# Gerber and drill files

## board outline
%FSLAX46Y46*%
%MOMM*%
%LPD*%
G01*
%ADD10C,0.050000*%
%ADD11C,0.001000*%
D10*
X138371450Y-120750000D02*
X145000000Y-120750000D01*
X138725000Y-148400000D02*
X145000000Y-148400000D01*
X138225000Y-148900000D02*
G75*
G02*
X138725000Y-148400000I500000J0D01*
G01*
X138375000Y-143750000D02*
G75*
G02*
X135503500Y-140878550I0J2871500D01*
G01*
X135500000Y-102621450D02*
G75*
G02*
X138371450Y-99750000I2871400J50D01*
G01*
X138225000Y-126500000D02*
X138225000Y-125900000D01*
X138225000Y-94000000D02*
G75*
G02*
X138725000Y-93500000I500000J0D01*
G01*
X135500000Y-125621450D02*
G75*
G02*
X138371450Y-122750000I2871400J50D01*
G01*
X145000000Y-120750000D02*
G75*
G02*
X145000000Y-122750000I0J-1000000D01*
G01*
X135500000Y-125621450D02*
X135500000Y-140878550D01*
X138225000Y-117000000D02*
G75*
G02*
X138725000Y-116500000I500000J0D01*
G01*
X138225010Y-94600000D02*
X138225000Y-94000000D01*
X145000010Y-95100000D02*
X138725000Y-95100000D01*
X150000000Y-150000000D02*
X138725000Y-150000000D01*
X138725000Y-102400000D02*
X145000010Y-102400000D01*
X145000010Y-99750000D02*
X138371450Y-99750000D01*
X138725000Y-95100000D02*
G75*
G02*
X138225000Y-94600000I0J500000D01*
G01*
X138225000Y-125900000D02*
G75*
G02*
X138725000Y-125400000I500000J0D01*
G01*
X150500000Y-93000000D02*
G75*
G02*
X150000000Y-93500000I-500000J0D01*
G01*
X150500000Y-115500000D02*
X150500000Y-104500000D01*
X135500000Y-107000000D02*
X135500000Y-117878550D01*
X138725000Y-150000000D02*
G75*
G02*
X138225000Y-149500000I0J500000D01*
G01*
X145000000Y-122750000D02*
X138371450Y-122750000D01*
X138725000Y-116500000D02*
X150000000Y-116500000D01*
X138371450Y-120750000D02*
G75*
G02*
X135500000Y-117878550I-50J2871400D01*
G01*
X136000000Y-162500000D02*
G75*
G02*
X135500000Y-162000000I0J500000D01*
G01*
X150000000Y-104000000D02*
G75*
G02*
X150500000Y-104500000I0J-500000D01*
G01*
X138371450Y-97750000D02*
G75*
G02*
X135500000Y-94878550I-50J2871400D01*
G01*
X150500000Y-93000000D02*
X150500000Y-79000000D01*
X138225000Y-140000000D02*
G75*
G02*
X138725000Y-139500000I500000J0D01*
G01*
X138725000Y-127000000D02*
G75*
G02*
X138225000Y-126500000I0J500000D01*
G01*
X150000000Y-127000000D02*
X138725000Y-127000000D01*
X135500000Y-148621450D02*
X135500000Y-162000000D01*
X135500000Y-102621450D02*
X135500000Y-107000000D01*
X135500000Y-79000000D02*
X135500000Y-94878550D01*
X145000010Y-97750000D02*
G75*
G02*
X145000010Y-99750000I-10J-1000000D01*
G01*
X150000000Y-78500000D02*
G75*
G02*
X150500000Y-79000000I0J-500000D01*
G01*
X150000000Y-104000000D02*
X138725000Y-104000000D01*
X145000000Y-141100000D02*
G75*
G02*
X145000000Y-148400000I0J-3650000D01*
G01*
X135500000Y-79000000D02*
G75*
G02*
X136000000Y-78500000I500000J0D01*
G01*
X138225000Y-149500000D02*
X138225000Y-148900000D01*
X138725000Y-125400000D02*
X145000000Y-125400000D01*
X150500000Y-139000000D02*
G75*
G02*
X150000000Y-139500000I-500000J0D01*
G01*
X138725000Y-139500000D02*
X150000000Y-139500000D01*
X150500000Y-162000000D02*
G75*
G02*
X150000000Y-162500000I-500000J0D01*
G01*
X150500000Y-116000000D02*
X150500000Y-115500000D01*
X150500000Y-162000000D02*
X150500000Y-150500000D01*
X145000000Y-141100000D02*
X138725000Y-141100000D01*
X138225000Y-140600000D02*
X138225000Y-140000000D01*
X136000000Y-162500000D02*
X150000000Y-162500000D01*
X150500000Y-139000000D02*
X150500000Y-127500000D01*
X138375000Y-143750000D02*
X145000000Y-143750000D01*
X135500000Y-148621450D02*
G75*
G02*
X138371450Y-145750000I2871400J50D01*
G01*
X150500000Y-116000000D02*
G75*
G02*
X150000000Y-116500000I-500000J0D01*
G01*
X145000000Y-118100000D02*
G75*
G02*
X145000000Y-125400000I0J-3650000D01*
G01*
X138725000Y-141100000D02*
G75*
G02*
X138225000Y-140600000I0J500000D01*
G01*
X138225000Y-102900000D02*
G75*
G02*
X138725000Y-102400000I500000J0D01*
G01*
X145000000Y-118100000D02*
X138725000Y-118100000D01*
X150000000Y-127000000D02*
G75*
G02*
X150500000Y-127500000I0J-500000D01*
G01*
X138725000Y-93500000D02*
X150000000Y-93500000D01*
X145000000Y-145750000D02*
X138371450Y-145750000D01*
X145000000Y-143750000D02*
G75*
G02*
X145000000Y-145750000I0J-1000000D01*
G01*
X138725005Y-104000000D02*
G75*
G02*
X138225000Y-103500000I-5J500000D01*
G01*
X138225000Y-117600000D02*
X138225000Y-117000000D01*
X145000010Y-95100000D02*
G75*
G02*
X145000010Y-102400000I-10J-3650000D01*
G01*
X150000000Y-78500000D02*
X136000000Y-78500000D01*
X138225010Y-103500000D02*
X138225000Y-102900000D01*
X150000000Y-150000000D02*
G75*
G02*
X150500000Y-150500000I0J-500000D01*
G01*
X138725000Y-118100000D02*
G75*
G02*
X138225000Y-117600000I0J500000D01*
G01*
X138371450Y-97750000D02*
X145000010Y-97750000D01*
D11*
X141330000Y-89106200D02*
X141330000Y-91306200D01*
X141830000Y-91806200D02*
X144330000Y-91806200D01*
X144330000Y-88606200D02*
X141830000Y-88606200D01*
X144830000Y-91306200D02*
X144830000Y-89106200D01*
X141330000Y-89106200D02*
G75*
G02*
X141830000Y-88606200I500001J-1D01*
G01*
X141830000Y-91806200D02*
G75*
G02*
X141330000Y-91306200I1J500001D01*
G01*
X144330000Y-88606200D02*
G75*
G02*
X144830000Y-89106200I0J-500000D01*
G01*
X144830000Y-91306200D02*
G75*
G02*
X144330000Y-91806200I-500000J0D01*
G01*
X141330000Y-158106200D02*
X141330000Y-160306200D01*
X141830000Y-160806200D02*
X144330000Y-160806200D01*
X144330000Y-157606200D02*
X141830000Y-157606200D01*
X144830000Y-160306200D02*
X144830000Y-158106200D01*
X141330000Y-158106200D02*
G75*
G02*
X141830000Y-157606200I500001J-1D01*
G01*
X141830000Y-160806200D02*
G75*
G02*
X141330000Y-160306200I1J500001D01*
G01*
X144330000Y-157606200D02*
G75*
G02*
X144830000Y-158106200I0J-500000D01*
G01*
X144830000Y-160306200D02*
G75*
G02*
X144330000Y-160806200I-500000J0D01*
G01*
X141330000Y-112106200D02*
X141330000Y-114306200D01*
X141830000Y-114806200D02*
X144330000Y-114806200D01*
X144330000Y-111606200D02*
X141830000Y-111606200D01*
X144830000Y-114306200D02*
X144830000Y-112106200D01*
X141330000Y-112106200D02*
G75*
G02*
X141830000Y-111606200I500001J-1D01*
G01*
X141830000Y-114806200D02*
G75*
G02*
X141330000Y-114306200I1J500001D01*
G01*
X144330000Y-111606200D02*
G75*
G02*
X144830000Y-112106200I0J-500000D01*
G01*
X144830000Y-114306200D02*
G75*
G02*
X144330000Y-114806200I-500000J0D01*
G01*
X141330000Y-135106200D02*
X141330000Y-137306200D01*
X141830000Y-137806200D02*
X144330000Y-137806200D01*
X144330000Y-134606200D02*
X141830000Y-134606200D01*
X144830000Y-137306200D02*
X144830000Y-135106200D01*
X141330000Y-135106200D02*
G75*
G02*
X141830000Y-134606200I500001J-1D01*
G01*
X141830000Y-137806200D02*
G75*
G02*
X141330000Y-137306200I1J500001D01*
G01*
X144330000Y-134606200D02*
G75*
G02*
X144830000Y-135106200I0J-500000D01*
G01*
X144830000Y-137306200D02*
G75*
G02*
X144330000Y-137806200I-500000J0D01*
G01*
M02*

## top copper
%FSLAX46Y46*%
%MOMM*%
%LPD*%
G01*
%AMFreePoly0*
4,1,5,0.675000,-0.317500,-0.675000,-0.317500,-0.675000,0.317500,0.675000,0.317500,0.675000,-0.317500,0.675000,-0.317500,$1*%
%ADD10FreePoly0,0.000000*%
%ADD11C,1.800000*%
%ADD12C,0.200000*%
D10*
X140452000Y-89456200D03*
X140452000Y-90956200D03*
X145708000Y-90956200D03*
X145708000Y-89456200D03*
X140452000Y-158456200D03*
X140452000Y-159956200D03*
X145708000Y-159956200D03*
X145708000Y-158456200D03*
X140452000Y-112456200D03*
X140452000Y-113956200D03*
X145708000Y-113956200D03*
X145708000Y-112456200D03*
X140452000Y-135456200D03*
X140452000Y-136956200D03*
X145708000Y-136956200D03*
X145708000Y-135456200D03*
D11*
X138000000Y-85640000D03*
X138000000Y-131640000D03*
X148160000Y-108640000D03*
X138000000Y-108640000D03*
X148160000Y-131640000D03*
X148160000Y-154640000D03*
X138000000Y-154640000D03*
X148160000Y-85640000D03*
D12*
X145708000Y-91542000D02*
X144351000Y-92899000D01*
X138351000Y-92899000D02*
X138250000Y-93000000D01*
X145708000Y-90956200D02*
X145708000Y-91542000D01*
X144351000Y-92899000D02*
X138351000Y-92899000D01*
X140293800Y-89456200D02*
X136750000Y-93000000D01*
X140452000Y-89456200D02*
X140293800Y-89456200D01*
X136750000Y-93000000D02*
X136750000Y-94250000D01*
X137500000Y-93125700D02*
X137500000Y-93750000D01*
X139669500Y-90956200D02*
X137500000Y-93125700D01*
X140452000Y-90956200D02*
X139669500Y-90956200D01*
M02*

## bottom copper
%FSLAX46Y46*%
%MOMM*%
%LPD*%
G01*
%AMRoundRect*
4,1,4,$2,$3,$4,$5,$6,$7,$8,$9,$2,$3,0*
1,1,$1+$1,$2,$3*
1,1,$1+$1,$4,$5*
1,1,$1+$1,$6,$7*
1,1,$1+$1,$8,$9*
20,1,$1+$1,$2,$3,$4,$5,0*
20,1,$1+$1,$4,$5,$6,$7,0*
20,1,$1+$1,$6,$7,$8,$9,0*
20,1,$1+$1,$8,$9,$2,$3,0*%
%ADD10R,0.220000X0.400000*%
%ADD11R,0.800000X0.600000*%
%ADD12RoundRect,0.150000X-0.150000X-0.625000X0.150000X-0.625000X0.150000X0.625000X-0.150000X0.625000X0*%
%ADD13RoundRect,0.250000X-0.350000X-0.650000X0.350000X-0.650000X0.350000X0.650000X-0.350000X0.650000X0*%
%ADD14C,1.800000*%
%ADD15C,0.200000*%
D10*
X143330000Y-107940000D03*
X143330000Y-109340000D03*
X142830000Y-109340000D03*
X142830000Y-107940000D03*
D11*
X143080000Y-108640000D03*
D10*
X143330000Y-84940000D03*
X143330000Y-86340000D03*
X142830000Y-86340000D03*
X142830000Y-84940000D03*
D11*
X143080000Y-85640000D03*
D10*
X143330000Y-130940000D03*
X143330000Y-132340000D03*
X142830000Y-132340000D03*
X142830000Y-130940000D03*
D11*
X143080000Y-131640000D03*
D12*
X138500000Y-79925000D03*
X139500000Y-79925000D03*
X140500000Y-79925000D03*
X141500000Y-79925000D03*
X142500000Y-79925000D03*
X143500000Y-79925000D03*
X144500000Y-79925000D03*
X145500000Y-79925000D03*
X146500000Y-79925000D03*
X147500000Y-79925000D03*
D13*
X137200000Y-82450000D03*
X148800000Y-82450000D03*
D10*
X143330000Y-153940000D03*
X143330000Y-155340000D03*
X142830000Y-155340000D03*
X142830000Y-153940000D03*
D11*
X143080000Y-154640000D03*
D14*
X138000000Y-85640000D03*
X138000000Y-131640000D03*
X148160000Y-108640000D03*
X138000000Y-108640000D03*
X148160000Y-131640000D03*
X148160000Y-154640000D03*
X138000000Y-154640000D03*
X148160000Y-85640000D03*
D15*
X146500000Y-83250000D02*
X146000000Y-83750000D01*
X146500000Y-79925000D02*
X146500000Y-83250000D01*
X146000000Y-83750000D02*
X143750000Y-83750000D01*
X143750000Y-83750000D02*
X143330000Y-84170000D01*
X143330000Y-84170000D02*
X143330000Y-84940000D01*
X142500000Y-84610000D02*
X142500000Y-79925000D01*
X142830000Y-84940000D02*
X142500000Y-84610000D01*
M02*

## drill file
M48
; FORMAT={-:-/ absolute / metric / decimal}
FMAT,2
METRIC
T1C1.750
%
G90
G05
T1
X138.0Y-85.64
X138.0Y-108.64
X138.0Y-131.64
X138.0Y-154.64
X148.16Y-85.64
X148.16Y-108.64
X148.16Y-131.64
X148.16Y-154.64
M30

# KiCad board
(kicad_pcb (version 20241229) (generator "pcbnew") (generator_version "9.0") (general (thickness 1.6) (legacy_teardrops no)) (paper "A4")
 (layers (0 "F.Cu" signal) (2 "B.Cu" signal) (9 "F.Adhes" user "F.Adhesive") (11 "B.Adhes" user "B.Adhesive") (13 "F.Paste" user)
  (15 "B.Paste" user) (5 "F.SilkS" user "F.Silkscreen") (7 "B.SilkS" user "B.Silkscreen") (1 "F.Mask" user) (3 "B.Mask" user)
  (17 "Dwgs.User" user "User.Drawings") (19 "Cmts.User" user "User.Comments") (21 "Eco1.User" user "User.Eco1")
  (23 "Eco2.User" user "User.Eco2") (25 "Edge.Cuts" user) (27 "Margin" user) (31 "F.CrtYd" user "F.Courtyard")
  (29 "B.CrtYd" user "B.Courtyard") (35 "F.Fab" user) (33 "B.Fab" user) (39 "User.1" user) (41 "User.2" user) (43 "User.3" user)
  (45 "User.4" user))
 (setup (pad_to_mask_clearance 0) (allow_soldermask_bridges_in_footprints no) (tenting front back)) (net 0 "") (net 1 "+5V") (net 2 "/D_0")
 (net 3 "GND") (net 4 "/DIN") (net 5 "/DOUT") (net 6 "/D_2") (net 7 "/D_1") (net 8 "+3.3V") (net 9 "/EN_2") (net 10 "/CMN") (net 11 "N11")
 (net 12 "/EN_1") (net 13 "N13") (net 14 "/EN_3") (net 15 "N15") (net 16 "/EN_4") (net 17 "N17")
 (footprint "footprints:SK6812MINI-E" (layer "F.Cu") (at 143.08 90.2062)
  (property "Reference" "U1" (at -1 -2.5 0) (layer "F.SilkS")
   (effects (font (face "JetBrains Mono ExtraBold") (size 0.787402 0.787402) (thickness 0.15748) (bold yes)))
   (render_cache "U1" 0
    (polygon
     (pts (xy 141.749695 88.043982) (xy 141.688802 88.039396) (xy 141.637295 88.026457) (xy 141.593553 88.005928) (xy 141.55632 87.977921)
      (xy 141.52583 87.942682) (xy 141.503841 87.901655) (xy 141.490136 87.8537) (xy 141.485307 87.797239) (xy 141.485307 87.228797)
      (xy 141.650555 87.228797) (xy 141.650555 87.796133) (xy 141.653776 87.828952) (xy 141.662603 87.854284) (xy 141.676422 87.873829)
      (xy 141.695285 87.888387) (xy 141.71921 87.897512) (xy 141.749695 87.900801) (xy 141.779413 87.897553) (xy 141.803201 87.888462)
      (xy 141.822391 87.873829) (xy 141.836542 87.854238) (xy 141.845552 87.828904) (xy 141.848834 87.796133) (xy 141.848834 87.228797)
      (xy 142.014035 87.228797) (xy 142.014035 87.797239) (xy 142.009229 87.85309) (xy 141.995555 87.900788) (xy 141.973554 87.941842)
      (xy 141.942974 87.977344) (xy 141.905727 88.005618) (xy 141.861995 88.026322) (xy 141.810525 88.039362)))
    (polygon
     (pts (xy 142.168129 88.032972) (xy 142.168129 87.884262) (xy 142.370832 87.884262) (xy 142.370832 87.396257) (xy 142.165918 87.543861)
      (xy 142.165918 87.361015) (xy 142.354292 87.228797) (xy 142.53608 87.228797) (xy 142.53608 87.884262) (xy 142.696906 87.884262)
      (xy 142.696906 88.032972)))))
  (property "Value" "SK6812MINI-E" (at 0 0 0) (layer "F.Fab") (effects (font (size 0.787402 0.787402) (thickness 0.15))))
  (fp_line (start -1.75 -1.1) (end -1.75 1.1) (stroke (width 0.001) (type solid)) (layer "Edge.Cuts"))
  (fp_line (start -1.25 1.6) (end 1.25 1.6) (stroke (width 0.001) (type solid)) (layer "Edge.Cuts"))
  (fp_line (start 1.25 -1.6) (end -1.25 -1.6) (stroke (width 0.001) (type solid)) (layer "Edge.Cuts"))
  (fp_line (start 1.75 1.1) (end 1.75 -1.1) (stroke (width 0.001) (type solid)) (layer "Edge.Cuts"))
  (fp_arc (start -1.75 -1.1) (mid -1.603553 -1.453553) (end -1.25 -1.6) (stroke (width 0.001) (type default)) (layer "Edge.Cuts"))
  (fp_arc (start -1.25 1.6) (mid -1.603553 1.453553) (end -1.75 1.1) (stroke (width 0.001) (type default)) (layer "Edge.Cuts"))
  (fp_arc (start 1.25 -1.6) (mid 1.603553 -1.453553) (end 1.75 -1.1) (stroke (width 0.001) (type default)) (layer "Edge.Cuts"))
  (fp_arc (start 1.75 1.1) (mid 1.603553 1.453553) (end 1.25 1.6) (stroke (width 0.001) (type default)) (layer "Edge.Cuts"))
  (pad "P$1" smd custom (at -2.628 -0.75) (size 1.35 0.635) (layers "F.Cu" "F.Mask" "F.Paste") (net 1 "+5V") (solder_mask_margin 0.102)
   (options (clearance outline) (anchor rect)) (primitives))
  (pad "P$2" smd custom (at -2.628 0.75) (size 1.35 0.635) (layers "F.Cu" "F.Mask" "F.Paste") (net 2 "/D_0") (solder_mask_margin 0.102)
   (options (clearance outline) (anchor rect)) (primitives))
  (pad "P$3" smd custom (at 2.628 0.75) (size 1.35 0.635) (layers "F.Cu" "F.Mask" "F.Paste") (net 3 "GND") (solder_mask_margin 0.102)
   (options (clearance outline) (anchor rect)) (primitives))
  (pad "P$4" smd custom (at 2.628 -0.75) (size 1.35 0.635) (layers "F.Cu" "F.Mask" "F.Paste") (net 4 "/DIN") (solder_mask_margin 0.102)
   (options (clearance outline) (anchor rect)) (primitives)))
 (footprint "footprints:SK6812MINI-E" (layer "F.Cu") (at 143.08 159.2062)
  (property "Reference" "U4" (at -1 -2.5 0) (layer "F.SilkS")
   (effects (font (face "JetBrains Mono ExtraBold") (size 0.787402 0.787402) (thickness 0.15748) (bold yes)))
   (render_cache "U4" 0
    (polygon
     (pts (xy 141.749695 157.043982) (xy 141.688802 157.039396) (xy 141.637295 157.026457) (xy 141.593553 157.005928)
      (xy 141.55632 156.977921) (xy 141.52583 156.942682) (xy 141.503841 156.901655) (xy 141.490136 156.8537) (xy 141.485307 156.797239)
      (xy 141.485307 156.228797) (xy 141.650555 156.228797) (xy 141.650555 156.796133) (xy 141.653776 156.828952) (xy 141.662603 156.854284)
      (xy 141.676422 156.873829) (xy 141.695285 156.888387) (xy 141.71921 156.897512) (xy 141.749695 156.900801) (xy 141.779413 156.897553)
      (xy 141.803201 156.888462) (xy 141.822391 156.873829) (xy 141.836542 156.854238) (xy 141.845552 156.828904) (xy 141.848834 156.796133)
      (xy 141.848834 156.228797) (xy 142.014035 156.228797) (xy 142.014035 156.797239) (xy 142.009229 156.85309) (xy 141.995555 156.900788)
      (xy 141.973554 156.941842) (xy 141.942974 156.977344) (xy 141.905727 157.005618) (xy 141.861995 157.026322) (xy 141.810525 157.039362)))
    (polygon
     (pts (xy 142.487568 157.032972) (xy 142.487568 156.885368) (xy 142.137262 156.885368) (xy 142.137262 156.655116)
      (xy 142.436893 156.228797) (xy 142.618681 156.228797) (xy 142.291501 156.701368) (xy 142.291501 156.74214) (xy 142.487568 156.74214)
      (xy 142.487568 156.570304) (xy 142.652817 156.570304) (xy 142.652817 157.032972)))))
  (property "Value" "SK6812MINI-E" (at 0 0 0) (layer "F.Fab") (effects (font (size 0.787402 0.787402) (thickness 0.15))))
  (fp_line (start -1.75 -1.1) (end -1.75 1.1) (stroke (width 0.001) (type solid)) (layer "Edge.Cuts"))
  (fp_line (start -1.25 1.6) (end 1.25 1.6) (stroke (width 0.001) (type solid)) (layer "Edge.Cuts"))
  (fp_line (start 1.25 -1.6) (end -1.25 -1.6) (stroke (width 0.001) (type solid)) (layer "Edge.Cuts"))
  (fp_line (start 1.75 1.1) (end 1.75 -1.1) (stroke (width 0.001) (type solid)) (layer "Edge.Cuts"))
  (fp_arc (start -1.75 -1.1) (mid -1.603553 -1.453553) (end -1.25 -1.6) (stroke (width 0.001) (type default)) (layer "Edge.Cuts"))
  (fp_arc (start -1.25 1.6) (mid -1.603553 1.453553) (end -1.75 1.1) (stroke (width 0.001) (type default)) (layer "Edge.Cuts"))
  (fp_arc (start 1.25 -1.6) (mid 1.603553 -1.453553) (end 1.75 -1.1) (stroke (width 0.001) (type default)) (layer "Edge.Cuts"))
  (fp_arc (start 1.75 1.1) (mid 1.603553 1.453553) (end 1.25 1.6) (stroke (width 0.001) (type default)) (layer "Edge.Cuts"))
  (pad "P$1" smd custom (at -2.628 -0.75) (size 1.35 0.635) (layers "F.Cu" "F.Mask" "F.Paste") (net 1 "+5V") (solder_mask_margin 0.102)
   (options (clearance outline) (anchor rect)) (primitives))
  (pad "P$2" smd custom (at -2.628 0.75) (size 1.35 0.635) (layers "F.Cu" "F.Mask" "F.Paste") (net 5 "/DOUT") (solder_mask_margin 0.102)
   (options (clearance outline) (anchor rect)) (primitives))
  (pad "P$3" smd custom (at 2.628 0.75) (size 1.35 0.635) (layers "F.Cu" "F.Mask" "F.Paste") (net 3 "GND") (solder_mask_margin 0.102)
   (options (clearance outline) (anchor rect)) (primitives))
  (pad "P$4" smd custom (at 2.628 -0.75) (size 1.35 0.635) (layers "F.Cu" "F.Mask" "F.Paste") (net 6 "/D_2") (solder_mask_margin 0.102)
   (options (clearance outline) (anchor rect)) (primitives)))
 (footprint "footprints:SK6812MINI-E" (layer "F.Cu") (at 143.08 113.2062)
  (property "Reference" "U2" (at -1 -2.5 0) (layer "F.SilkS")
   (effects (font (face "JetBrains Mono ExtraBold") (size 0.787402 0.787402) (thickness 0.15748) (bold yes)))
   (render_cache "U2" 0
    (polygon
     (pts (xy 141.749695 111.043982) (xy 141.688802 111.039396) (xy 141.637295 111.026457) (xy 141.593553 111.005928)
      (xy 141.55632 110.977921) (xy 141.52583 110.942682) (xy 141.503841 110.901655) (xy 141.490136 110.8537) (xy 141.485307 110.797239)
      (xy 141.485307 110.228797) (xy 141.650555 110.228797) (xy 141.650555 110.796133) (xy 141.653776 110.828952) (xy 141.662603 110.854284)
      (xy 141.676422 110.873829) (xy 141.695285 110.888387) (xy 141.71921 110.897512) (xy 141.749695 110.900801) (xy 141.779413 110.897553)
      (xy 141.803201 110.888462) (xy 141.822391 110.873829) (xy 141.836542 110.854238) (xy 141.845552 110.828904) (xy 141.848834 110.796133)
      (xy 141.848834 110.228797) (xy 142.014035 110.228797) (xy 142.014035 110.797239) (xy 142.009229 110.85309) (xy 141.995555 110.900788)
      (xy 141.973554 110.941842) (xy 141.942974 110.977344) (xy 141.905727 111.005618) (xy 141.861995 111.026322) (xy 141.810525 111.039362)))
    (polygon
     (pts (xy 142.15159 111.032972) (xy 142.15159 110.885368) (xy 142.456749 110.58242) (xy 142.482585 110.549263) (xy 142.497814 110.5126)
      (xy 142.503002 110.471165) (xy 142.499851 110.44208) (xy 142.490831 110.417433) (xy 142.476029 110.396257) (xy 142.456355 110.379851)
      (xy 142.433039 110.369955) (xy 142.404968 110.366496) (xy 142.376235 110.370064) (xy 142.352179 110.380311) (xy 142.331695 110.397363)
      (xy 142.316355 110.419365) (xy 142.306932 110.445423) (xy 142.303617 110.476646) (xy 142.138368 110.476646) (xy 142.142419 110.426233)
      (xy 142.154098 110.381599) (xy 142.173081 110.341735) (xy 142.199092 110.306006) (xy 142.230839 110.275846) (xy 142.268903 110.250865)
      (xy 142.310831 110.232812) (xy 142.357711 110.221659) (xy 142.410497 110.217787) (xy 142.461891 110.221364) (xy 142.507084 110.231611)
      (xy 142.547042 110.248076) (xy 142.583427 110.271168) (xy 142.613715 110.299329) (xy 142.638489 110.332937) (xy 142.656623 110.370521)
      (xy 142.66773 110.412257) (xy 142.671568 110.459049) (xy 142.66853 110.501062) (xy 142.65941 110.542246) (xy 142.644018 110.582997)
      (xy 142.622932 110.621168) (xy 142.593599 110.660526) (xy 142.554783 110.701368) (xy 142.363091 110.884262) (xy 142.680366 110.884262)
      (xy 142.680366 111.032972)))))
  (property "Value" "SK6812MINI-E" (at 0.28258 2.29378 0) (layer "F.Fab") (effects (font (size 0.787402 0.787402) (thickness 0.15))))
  (fp_line (start -1.75 -1.1) (end -1.75 1.1) (stroke (width 0.001) (type solid)) (layer "Edge.Cuts"))
  (fp_line (start -1.25 1.6) (end 1.25 1.6) (stroke (width 0.001) (type solid)) (layer "Edge.Cuts"))
  (fp_line (start 1.25 -1.6) (end -1.25 -1.6) (stroke (width 0.001) (type solid)) (layer "Edge.Cuts"))
  (fp_line (start 1.75 1.1) (end 1.75 -1.1) (stroke (width 0.001) (type solid)) (layer "Edge.Cuts"))
  (fp_arc (start -1.75 -1.1) (mid -1.603553 -1.453553) (end -1.25 -1.6) (stroke (width 0.001) (type default)) (layer "Edge.Cuts"))
  (fp_arc (start -1.25 1.6) (mid -1.603553 1.453553) (end -1.75 1.1) (stroke (width 0.001) (type default)) (layer "Edge.Cuts"))
  (fp_arc (start 1.25 -1.6) (mid 1.603553 -1.453553) (end 1.75 -1.1) (stroke (width 0.001) (type default)) (layer "Edge.Cuts"))
  (fp_arc (start 1.75 1.1) (mid 1.603553 1.453553) (end 1.25 1.6) (stroke (width 0.001) (type default)) (layer "Edge.Cuts"))
  (pad "P$1" smd custom (at -2.628 -0.75) (size 1.35 0.635) (layers "F.Cu" "F.Mask" "F.Paste") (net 1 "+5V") (solder_mask_margin 0.102)
   (options (clearance outline) (anchor rect)) (primitives))
  (pad "P$2" smd custom (at -2.628 0.75) (size 1.35 0.635) (layers "F.Cu" "F.Mask" "F.Paste") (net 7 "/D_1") (solder_mask_margin 0.102)
   (options (clearance outline) (anchor rect)) (primitives))
  (pad "P$3" smd custom (at 2.628 0.75) (size 1.35 0.635) (layers "F.Cu" "F.Mask" "F.Paste") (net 3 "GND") (solder_mask_margin 0.102)
   (options (clearance outline) (anchor rect)) (primitives))
  (pad "P$4" smd custom (at 2.628 -0.75) (size 1.35 0.635) (layers "F.Cu" "F.Mask" "F.Paste") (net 2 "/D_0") (solder_mask_margin 0.102)
   (options (clearance outline) (anchor rect)) (primitives)))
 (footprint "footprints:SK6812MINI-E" (layer "F.Cu") (at 143.08 136.2062)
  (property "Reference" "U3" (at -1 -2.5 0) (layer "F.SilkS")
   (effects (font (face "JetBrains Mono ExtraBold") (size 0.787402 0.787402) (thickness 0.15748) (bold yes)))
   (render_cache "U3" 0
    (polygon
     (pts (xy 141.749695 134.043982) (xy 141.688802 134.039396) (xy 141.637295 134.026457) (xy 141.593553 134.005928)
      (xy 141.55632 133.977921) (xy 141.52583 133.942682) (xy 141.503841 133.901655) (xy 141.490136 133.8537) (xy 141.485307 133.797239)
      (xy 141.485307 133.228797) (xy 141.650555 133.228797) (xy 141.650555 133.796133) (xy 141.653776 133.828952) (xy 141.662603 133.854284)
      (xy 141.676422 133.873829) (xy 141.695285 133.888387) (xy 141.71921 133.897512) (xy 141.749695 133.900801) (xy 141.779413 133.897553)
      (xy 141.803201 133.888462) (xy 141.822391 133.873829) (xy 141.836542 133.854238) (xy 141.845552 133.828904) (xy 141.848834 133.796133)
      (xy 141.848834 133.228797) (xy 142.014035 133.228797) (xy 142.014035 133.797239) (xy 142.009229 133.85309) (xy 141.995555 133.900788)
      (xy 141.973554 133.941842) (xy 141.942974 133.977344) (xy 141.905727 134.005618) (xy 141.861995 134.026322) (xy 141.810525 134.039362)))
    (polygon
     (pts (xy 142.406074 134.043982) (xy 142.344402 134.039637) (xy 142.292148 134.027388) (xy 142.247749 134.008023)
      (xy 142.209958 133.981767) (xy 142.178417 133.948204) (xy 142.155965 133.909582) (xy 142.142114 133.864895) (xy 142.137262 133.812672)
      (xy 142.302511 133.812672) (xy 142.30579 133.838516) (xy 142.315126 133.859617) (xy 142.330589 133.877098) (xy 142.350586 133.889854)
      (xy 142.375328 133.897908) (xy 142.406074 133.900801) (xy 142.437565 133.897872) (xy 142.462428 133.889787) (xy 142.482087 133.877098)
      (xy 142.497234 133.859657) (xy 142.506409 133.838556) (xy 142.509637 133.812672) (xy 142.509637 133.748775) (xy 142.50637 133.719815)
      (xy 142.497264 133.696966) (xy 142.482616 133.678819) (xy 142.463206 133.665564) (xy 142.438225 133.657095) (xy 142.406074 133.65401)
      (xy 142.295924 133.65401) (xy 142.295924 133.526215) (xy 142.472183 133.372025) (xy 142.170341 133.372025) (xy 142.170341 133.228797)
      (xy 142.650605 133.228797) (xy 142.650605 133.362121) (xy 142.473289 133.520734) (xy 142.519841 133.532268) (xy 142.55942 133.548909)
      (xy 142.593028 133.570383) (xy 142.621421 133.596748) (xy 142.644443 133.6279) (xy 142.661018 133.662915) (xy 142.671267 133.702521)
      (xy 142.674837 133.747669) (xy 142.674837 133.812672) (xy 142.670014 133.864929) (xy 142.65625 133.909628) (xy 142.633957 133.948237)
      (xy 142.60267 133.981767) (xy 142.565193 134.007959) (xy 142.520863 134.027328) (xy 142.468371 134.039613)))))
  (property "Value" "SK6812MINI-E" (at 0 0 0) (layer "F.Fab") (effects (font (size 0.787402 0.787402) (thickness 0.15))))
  (fp_line (start -1.75 -1.1) (end -1.75 1.1) (stroke (width 0.001) (type solid)) (layer "Edge.Cuts"))
  (fp_line (start -1.25 1.6) (end 1.25 1.6) (stroke (width 0.001) (type solid)) (layer "Edge.Cuts"))
  (fp_line (start 1.25 -1.6) (end -1.25 -1.6) (stroke (width 0.001) (type solid)) (layer "Edge.Cuts"))
  (fp_line (start 1.75 1.1) (end 1.75 -1.1) (stroke (width 0.001) (type solid)) (layer "Edge.Cuts"))
  (fp_arc (start -1.75 -1.1) (mid -1.603553 -1.453553) (end -1.25 -1.6) (stroke (width 0.001) (type default)) (layer "Edge.Cuts"))
  (fp_arc (start -1.25 1.6) (mid -1.603553 1.453553) (end -1.75 1.1) (stroke (width 0.001) (type default)) (layer "Edge.Cuts"))
  (fp_arc (start 1.25 -1.6) (mid 1.603553 -1.453553) (end 1.75 -1.1) (stroke (width 0.001) (type default)) (layer "Edge.Cuts"))
  (fp_arc (start 1.75 1.1) (mid 1.603553 1.453553) (end 1.25 1.6) (stroke (width 0.001) (type default)) (layer "Edge.Cuts"))
  (pad "P$1" smd custom (at -2.628 -0.75) (size 1.35 0.635) (layers "F.Cu" "F.Mask" "F.Paste") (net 1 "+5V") (solder_mask_margin 0.102)
   (options (clearance outline) (anchor rect)) (primitives))
  (pad "P$2" smd custom (at -2.628 0.75) (size 1.35 0.635) (layers "F.Cu" "F.Mask" "F.Paste") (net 6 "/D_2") (solder_mask_margin 0.102)
   (options (clearance outline) (anchor rect)) (primitives))
  (pad "P$3" smd custom (at 2.628 0.75) (size 1.35 0.635) (layers "F.Cu" "F.Mask" "F.Paste") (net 3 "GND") (solder_mask_margin 0.102)
   (options (clearance outline) (anchor rect)) (primitives))
  (pad "P$4" smd custom (at 2.628 -0.75) (size 1.35 0.635) (layers "F.Cu" "F.Mask" "F.Paste") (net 7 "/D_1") (solder_mask_margin 0.102)
   (options (clearance outline) (anchor rect)) (primitives)))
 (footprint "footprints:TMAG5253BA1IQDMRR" (layer "B.Cu") (at 143.08 108.64 180)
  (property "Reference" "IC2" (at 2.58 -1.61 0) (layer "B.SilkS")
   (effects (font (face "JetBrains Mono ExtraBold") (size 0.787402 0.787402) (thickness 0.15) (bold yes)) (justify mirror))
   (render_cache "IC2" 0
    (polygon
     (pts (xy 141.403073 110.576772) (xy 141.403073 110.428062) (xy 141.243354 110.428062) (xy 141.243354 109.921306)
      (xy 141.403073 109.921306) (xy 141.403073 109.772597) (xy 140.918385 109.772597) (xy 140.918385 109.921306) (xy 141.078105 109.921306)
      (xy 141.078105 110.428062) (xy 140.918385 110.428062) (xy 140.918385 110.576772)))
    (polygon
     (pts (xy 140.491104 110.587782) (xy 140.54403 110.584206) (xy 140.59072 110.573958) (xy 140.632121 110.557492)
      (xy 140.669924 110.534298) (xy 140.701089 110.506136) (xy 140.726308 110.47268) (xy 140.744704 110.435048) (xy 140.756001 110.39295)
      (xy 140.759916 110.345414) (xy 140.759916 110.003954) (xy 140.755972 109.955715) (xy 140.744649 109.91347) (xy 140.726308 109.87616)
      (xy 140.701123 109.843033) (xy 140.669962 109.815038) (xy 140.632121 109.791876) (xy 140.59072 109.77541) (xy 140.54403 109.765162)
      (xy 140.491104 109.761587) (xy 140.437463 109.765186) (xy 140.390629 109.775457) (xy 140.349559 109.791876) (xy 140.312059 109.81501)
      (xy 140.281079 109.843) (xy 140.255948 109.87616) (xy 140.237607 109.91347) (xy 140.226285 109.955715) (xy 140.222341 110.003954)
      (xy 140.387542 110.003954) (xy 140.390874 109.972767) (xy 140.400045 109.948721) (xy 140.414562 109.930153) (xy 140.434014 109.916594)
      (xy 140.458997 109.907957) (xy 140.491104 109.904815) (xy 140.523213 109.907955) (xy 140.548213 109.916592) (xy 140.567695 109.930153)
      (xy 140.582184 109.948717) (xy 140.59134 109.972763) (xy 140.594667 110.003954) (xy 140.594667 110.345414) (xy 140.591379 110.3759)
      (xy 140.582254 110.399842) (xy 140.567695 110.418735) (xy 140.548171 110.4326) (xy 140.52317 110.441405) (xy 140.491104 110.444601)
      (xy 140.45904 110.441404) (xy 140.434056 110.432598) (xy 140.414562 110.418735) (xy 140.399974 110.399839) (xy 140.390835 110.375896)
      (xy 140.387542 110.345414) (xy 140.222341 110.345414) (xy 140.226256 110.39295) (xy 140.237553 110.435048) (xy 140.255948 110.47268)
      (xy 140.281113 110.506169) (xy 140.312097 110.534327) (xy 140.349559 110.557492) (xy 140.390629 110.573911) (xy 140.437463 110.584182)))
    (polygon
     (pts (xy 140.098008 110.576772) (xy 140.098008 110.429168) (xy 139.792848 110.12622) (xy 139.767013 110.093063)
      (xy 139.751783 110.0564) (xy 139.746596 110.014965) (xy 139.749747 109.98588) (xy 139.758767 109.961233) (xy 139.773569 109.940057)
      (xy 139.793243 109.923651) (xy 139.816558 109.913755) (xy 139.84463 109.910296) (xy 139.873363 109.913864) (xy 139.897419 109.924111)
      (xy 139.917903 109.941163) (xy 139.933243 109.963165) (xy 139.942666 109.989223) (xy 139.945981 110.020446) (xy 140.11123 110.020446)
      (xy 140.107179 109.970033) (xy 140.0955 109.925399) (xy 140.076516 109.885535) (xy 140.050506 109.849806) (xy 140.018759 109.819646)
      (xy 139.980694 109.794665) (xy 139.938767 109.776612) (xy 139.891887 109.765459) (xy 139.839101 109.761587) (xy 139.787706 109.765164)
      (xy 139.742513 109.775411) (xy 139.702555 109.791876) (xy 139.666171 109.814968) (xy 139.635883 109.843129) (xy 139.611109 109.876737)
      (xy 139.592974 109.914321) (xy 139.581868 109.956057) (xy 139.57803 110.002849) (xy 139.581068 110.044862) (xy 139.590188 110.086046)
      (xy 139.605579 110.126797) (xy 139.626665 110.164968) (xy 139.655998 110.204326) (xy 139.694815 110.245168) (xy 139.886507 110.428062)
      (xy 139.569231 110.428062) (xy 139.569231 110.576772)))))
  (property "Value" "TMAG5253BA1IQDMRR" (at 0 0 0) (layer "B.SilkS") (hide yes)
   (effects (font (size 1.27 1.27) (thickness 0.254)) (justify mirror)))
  (pad "1" smd rect (at -0.25 0.7 180) (size 0.22 0.4) (layers "B.Cu" "B.Mask" "B.Paste") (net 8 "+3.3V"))
  (pad "2" smd rect (at -0.25 -0.7 180) (size 0.22 0.4) (layers "B.Cu" "B.Mask" "B.Paste") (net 3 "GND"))
  (pad "3" smd rect (at 0.25 -0.7 180) (size 0.22 0.4) (layers "B.Cu" "B.Mask" "B.Paste") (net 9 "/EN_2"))
  (pad "4" smd rect (at 0.25 0.7 180) (size 0.22 0.4) (layers "B.Cu" "B.Mask" "B.Paste") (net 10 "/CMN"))
  (pad "5" smd rect (at 0 0 90) (size 0.6 0.8) (layers "B.Cu" "B.Mask" "B.Paste") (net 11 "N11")))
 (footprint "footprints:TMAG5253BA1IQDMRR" (layer "B.Cu") (at 143.08 85.64 180)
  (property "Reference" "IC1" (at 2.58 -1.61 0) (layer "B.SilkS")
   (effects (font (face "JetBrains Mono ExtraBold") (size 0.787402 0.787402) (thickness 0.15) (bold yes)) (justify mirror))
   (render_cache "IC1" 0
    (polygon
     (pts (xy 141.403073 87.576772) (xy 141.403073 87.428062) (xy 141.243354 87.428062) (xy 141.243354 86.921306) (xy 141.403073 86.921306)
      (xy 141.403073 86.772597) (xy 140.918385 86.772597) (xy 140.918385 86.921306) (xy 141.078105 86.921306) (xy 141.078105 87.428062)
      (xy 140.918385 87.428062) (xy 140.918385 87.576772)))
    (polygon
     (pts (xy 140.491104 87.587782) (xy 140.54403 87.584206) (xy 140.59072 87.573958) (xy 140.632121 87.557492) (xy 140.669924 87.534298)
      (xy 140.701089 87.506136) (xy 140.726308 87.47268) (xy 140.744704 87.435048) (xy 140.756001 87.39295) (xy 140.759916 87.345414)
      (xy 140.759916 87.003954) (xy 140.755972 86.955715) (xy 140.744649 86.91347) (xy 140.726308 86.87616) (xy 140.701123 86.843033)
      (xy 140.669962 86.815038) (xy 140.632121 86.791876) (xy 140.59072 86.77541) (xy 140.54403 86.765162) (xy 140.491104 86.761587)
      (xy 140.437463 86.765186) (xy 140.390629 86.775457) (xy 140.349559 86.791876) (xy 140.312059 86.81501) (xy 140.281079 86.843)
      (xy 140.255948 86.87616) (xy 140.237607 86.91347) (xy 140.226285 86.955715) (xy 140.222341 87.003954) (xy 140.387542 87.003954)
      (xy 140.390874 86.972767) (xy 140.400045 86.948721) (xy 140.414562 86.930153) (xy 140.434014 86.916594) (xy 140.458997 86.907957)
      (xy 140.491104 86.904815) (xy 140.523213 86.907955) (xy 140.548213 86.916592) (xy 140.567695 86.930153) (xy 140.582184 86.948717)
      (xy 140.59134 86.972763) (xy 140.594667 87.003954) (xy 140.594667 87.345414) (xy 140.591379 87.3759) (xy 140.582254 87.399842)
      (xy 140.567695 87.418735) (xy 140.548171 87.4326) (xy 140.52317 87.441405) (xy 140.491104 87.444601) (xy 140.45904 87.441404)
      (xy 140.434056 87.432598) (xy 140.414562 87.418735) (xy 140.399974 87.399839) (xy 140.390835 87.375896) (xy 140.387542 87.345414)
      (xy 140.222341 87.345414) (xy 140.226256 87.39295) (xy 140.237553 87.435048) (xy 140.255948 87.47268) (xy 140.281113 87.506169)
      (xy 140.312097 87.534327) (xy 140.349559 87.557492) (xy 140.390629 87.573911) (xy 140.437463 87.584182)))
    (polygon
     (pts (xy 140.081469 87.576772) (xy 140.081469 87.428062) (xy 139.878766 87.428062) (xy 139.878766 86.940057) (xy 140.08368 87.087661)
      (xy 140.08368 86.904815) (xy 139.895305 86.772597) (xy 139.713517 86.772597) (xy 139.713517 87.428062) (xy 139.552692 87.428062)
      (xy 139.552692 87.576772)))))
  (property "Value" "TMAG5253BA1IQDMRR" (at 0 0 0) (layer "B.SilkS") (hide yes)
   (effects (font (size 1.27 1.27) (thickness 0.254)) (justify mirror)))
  (pad "1" smd rect (at -0.25 0.7 180) (size 0.22 0.4) (layers "B.Cu" "B.Mask" "B.Paste") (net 8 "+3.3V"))
  (pad "2" smd rect (at -0.25 -0.7 180) (size 0.22 0.4) (layers "B.Cu" "B.Mask" "B.Paste") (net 3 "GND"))
  (pad "3" smd rect (at 0.25 -0.7 180) (size 0.22 0.4) (layers "B.Cu" "B.Mask" "B.Paste") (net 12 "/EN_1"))
  (pad "4" smd rect (at 0.25 0.7 180) (size 0.22 0.4) (layers "B.Cu" "B.Mask" "B.Paste") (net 10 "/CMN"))
  (pad "5" smd rect (at 0 0 90) (size 0.6 0.8) (layers "B.Cu" "B.Mask" "B.Paste") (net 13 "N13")))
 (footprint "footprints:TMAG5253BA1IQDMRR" (layer "B.Cu") (at 143.08 131.64 180)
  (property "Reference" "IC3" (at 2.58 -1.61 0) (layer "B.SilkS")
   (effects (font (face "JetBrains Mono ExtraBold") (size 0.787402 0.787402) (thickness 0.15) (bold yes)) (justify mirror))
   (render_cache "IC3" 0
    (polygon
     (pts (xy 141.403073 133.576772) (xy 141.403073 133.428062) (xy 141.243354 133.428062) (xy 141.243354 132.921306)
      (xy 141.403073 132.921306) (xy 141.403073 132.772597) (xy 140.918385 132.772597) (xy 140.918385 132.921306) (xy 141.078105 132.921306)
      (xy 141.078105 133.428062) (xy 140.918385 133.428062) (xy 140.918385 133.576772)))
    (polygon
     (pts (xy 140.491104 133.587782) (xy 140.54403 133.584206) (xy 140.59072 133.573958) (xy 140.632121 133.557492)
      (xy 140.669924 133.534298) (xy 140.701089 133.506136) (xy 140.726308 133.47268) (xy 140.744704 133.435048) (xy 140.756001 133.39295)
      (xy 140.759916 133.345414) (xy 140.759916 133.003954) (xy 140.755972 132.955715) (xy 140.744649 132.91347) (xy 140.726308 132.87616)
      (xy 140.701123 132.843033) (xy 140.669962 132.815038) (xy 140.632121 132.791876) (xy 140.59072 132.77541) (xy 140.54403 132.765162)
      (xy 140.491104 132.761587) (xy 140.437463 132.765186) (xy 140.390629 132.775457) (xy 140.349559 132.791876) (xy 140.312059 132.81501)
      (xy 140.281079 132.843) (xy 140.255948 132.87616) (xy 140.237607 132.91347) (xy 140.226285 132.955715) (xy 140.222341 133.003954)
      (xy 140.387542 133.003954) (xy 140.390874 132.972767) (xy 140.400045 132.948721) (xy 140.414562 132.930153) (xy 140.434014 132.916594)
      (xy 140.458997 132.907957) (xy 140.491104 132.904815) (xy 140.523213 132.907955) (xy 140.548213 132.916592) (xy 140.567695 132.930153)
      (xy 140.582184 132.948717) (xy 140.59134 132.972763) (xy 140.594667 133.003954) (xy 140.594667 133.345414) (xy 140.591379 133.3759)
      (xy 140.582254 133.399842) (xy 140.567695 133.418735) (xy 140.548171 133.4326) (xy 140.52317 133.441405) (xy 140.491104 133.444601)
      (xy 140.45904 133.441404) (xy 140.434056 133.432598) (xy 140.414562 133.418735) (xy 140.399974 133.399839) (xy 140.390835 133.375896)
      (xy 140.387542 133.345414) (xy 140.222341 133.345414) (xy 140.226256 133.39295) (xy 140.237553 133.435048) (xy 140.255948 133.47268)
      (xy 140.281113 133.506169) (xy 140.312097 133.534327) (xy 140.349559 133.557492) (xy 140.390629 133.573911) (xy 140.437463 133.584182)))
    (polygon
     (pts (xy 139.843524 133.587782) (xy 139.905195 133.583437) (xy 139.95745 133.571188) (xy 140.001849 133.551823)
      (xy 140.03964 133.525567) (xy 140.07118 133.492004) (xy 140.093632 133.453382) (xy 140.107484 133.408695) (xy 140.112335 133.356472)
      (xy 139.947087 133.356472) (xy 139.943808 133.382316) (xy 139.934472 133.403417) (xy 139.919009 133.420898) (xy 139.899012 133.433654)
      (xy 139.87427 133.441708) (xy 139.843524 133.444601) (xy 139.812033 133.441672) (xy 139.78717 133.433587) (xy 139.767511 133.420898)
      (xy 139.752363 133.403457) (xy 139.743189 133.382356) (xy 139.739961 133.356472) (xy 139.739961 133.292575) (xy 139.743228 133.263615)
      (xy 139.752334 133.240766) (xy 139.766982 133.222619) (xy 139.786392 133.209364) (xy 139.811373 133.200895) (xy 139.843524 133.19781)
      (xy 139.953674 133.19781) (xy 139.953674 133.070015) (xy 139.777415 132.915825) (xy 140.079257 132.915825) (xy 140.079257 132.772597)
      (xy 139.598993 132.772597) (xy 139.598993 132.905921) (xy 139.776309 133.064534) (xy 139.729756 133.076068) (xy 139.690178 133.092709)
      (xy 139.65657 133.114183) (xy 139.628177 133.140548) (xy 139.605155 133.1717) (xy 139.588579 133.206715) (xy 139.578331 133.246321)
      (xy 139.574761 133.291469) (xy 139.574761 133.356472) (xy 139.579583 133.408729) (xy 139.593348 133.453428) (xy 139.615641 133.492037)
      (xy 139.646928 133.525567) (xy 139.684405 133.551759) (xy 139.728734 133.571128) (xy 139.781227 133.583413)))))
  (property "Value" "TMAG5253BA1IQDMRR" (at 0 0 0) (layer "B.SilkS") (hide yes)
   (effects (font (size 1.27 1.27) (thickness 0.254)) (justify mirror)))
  (pad "1" smd rect (at -0.25 0.7 180) (size 0.22 0.4) (layers "B.Cu" "B.Mask" "B.Paste") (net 8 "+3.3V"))
  (pad "2" smd rect (at -0.25 -0.7 180) (size 0.22 0.4) (layers "B.Cu" "B.Mask" "B.Paste") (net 3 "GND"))
  (pad "3" smd rect (at 0.25 -0.7 180) (size 0.22 0.4) (layers "B.Cu" "B.Mask" "B.Paste") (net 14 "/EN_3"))
  (pad "4" smd rect (at 0.25 0.7 180) (size 0.22 0.4) (layers "B.Cu" "B.Mask" "B.Paste") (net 10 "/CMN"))
  (pad "5" smd rect (at 0 0 90) (size 0.6 0.8) (layers "B.Cu" "B.Mask" "B.Paste") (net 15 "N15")))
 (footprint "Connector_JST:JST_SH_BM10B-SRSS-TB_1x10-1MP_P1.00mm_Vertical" (layer "B.Cu") (at 143 81.25)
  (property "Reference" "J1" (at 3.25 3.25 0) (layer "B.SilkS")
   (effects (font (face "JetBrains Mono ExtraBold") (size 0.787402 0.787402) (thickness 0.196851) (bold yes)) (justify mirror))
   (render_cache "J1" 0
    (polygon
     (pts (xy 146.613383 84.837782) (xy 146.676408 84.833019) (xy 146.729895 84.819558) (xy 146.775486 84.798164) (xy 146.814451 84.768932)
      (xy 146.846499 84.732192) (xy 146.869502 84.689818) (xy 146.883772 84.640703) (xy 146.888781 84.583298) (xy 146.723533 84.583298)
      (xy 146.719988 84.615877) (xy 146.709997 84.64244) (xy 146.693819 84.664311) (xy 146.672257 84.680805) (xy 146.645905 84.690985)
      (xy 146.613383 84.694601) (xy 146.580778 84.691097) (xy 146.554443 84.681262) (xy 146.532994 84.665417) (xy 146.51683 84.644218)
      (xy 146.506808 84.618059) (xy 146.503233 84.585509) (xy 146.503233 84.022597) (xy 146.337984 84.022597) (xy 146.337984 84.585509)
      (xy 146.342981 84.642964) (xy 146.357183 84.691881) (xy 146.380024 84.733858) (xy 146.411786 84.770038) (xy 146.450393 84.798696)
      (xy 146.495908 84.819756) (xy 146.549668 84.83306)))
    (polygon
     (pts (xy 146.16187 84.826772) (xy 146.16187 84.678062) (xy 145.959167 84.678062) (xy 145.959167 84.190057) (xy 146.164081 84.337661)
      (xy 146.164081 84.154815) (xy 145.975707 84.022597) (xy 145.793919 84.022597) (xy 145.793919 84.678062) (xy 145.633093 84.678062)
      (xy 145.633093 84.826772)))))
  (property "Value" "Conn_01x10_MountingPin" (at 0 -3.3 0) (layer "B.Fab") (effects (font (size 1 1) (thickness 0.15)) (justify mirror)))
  (pad "1" smd roundrect (at -4.5 -1.325) (size 0.6 1.55) (layers "B.Cu" "B.Mask" "B.Paste") (roundrect_rratio 0.25) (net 12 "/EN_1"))
  (pad "2" smd roundrect (at -3.5 -1.325) (size 0.6 1.55) (layers "B.Cu" "B.Mask" "B.Paste") (roundrect_rratio 0.25) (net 9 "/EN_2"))
  (pad "3" smd roundrect (at -2.5 -1.325) (size 0.6 1.55) (layers "B.Cu" "B.Mask" "B.Paste") (roundrect_rratio 0.25) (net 14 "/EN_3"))
  (pad "4" smd roundrect (at -1.5 -1.325) (size 0.6 1.55) (layers "B.Cu" "B.Mask" "B.Paste") (roundrect_rratio 0.25) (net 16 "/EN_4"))
  (pad "5" smd roundrect (at -0.5 -1.325) (size 0.6 1.55) (layers "B.Cu" "B.Mask" "B.Paste") (roundrect_rratio 0.25) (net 10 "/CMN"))
  (pad "6" smd roundrect (at 0.5 -1.325) (size 0.6 1.55) (layers "B.Cu" "B.Mask" "B.Paste") (roundrect_rratio 0.25) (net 5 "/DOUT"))
  (pad "7" smd roundrect (at 1.5 -1.325) (size 0.6 1.55) (layers "B.Cu" "B.Mask" "B.Paste") (roundrect_rratio 0.25) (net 4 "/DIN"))
  (pad "8" smd roundrect (at 2.5 -1.325) (size 0.6 1.55) (layers "B.Cu" "B.Mask" "B.Paste") (roundrect_rratio 0.25) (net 1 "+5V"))
  (pad "9" smd roundrect (at 3.5 -1.325) (size 0.6 1.55) (layers "B.Cu" "B.Mask" "B.Paste") (roundrect_rratio 0.25) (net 8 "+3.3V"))
  (pad "10" smd roundrect (at 4.5 -1.325) (size 0.6 1.55) (layers "B.Cu" "B.Mask" "B.Paste") (roundrect_rratio 0.25) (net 3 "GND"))
  (pad "MP" smd roundrect (at -5.8 1.2) (size 1.2 1.8) (layers "B.Cu" "B.Mask" "B.Paste") (roundrect_rratio 0.208333) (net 3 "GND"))
  (pad "MP" smd roundrect (at 5.8 1.2) (size 1.2 1.8) (layers "B.Cu" "B.Mask" "B.Paste") (roundrect_rratio 0.208333) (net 3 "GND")))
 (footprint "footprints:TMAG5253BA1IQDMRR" (layer "B.Cu") (at 143.08 154.64 180)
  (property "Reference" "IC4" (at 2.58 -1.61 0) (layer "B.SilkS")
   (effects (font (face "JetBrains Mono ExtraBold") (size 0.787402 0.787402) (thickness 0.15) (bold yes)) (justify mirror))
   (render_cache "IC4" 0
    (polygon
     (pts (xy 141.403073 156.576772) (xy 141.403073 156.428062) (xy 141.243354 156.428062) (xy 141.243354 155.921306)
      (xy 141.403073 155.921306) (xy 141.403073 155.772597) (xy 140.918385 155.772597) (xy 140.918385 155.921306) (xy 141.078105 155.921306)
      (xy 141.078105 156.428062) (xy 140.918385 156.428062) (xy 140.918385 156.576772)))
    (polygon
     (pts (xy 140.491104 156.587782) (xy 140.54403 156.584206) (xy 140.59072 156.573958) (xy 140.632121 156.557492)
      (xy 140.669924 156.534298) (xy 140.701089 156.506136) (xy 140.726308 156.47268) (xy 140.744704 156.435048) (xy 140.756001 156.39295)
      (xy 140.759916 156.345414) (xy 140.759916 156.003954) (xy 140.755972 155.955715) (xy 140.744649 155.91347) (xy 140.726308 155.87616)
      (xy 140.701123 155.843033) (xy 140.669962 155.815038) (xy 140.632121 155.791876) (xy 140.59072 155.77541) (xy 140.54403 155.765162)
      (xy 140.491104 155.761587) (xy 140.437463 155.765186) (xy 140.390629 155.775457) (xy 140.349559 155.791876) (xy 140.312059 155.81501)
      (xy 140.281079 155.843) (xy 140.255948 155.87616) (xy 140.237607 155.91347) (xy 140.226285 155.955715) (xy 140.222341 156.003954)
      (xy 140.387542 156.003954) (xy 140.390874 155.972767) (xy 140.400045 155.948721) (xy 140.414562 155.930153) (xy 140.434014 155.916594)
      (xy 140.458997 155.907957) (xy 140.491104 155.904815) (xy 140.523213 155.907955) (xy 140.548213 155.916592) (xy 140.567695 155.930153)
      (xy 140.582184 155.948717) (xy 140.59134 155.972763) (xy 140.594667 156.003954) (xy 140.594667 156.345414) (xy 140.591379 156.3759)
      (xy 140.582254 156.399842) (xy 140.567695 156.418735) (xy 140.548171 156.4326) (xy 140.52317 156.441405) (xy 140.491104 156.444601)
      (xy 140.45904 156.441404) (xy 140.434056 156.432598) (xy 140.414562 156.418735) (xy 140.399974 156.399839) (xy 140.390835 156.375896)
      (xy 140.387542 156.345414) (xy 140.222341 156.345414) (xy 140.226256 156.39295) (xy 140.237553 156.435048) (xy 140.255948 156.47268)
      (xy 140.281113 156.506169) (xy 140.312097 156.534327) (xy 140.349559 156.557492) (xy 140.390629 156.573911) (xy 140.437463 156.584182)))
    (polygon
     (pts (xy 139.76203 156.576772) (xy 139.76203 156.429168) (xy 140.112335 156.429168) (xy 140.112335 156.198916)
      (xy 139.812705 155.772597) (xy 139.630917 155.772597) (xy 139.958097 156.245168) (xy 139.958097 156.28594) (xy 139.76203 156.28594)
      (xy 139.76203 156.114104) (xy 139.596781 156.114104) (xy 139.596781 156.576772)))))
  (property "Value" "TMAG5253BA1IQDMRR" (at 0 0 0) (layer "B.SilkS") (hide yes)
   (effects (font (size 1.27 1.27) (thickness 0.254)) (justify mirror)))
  (pad "1" smd rect (at -0.25 0.7 180) (size 0.22 0.4) (layers "B.Cu" "B.Mask" "B.Paste") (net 8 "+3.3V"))
  (pad "2" smd rect (at -0.25 -0.7 180) (size 0.22 0.4) (layers "B.Cu" "B.Mask" "B.Paste") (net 3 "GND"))
  (pad "3" smd rect (at 0.25 -0.7 180) (size 0.22 0.4) (layers "B.Cu" "B.Mask" "B.Paste") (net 16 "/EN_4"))
  (pad "4" smd rect (at 0.25 0.7 180) (size 0.22 0.4) (layers "B.Cu" "B.Mask" "B.Paste") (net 10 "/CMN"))
  (pad "5" smd rect (at 0 0 90) (size 0.6 0.8) (layers "B.Cu" "B.Mask" "B.Paste") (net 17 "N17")))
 (gr_line (start 138.37145 120.75) (end 145 120.75) (stroke (width 0.05) (type solid)) (layer "Edge.Cuts"))
 (gr_line (start 138.725 148.4) (end 145 148.4) (stroke (width 0.05) (type solid)) (layer "Edge.Cuts"))
 (gr_arc (start 138.225 148.9) (mid 138.371447 148.546447) (end 138.725 148.4) (stroke (width 0.05) (type solid)) (layer "Edge.Cuts"))
 (gr_arc (start 138.375 143.75) (mid 136.344596 142.908969) (end 135.50355 140.87855) (stroke (width 0.05) (type solid)) (layer "Edge.Cuts"))
 (gr_arc (start 135.5 102.62145) (mid 136.341014 100.591014) (end 138.37145 99.75) (stroke (width 0.05) (type solid)) (layer "Edge.Cuts"))
 (gr_line (start 138.225 126.5) (end 138.225 125.9) (stroke (width 0.05) (type solid)) (layer "Edge.Cuts"))
 (gr_arc (start 138.225 94) (mid 138.371447 93.646447) (end 138.725 93.5) (stroke (width 0.05) (type solid)) (layer "Edge.Cuts"))
 (gr_arc (start 135.5 125.62145) (mid 136.341014 123.591014) (end 138.37145 122.75) (stroke (width 0.05) (type solid)) (layer "Edge.Cuts"))
 (gr_arc (start 145 120.75) (mid 146 121.75) (end 145 122.75) (stroke (width 0.05) (type solid)) (layer "Edge.Cuts"))
 (gr_line (start 135.5 125.62145) (end 135.5 140.87855) (stroke (width 0.05) (type solid)) (layer "Edge.Cuts"))
 (gr_arc (start 138.225 117) (mid 138.371447 116.646447) (end 138.725 116.5) (stroke (width 0.05) (type solid)) (layer "Edge.Cuts"))
 (gr_line (start 138.22501 94.6) (end 138.225 94) (stroke (width 0.05) (type solid)) (layer "Edge.Cuts"))
 (gr_line (start 145.00001 95.1) (end 138.725 95.1) (stroke (width 0.05) (type solid)) (layer "Edge.Cuts"))
 (gr_line (start 150 150) (end 138.725 150) (stroke (width 0.05) (type solid)) (layer "Edge.Cuts"))
 (gr_line (start 138.725 102.4) (end 145.00001 102.4) (stroke (width 0.05) (type solid)) (layer "Edge.Cuts"))
 (gr_line (start 145.00001 99.75) (end 138.37145 99.75) (stroke (width 0.05) (type solid)) (layer "Edge.Cuts"))
 (gr_arc (start 138.725 95.1) (mid 138.371447 94.953553) (end 138.225 94.6) (stroke (width 0.05) (type solid)) (layer "Edge.Cuts"))
 (gr_arc (start 138.225 125.9) (mid 138.371447 125.546447) (end 138.725 125.4) (stroke (width 0.05) (type solid)) (layer "Edge.Cuts"))
 (gr_arc (start 150.5 93) (mid 150.353553 93.353553) (end 150 93.5) (stroke (width 0.05) (type solid)) (layer "Edge.Cuts"))
 (gr_line (start 150.5 115.5) (end 150.5 104.5) (stroke (width 0.05) (type solid)) (layer "Edge.Cuts"))
 (gr_line (start 135.5 107) (end 135.5 117.87855) (stroke (width 0.05) (type solid)) (layer "Edge.Cuts"))
 (gr_arc (start 138.725 150) (mid 138.371447 149.853553) (end 138.225 149.5) (stroke (width 0.05) (type solid)) (layer "Edge.Cuts"))
 (gr_line (start 145 122.75) (end 138.37145 122.75) (stroke (width 0.05) (type solid)) (layer "Edge.Cuts"))
 (gr_line (start 138.725 116.5) (end 150 116.5) (stroke (width 0.05) (type solid)) (layer "Edge.Cuts"))
 (gr_arc (start 138.37145 120.75) (mid 136.341014 119.908986) (end 135.5 117.87855) (stroke (width 0.05) (type solid)) (layer "Edge.Cuts"))
 (gr_arc (start 136 162.5) (mid 135.646447 162.353553) (end 135.5 162) (stroke (width 0.05) (type solid)) (layer "Edge.Cuts"))
 (gr_arc (start 150 104) (mid 150.353553 104.146447) (end 150.5 104.5) (stroke (width 0.05) (type solid)) (layer "Edge.Cuts"))
 (gr_arc (start 138.37145 97.75) (mid 136.341014 96.908986) (end 135.5 94.87855) (stroke (width 0.05) (type solid)) (layer "Edge.Cuts"))
 (gr_line (start 150.5 93) (end 150.5 79) (stroke (width 0.05) (type solid)) (layer "Edge.Cuts"))
 (gr_arc (start 138.225 140) (mid 138.371447 139.646447) (end 138.725 139.5) (stroke (width 0.05) (type solid)) (layer "Edge.Cuts"))
 (gr_arc (start 138.725 127) (mid 138.371447 126.853553) (end 138.225 126.5) (stroke (width 0.05) (type solid)) (layer "Edge.Cuts"))
 (gr_line (start 150 127) (end 138.725 127) (stroke (width 0.05) (type solid)) (layer "Edge.Cuts"))
 (gr_line (start 135.5 148.62145) (end 135.5 162) (stroke (width 0.05) (type solid)) (layer "Edge.Cuts"))
 (gr_line (start 135.5 102.62145) (end 135.5 107) (stroke (width 0.05) (type solid)) (layer "Edge.Cuts"))
 (gr_line (start 135.5 79) (end 135.5 94.87855) (stroke (width 0.05) (type solid)) (layer "Edge.Cuts"))
 (gr_arc (start 145.00001 97.75) (mid 146 98.75) (end 145.00001 99.75) (stroke (width 0.05) (type solid)) (layer "Edge.Cuts"))
 (gr_arc (start 150 78.5) (mid 150.353553 78.646447) (end 150.5 79) (stroke (width 0.05) (type solid)) (layer "Edge.Cuts"))
 (gr_line (start 150 104) (end 138.725 104) (stroke (width 0.05) (type solid)) (layer "Edge.Cuts"))
 (gr_arc (start 145 141.1) (mid 148.65 144.75) (end 145 148.4) (stroke (width 0.05) (type solid)) (layer "Edge.Cuts"))
 (gr_arc (start 135.5 79) (mid 135.646447 78.646447) (end 136 78.5) (stroke (width 0.05) (type solid)) (layer "Edge.Cuts"))
 (gr_line (start 138.225 149.5) (end 138.225 148.9) (stroke (width 0.05) (type solid)) (layer "Edge.Cuts"))
 (gr_line (start 138.725 125.4) (end 145 125.4) (stroke (width 0.05) (type solid)) (layer "Edge.Cuts"))
 (gr_arc (start 150.5 139) (mid 150.353553 139.353553) (end 150 139.5) (stroke (width 0.05) (type solid)) (layer "Edge.Cuts"))
 (gr_line (start 138.725 139.5) (end 150 139.5) (stroke (width 0.05) (type solid)) (layer "Edge.Cuts"))
 (gr_arc (start 150.5 162) (mid 150.353553 162.353553) (end 150 162.5) (stroke (width 0.05) (type solid)) (layer "Edge.Cuts"))
 (gr_line (start 150.5 116) (end 150.5 115.5) (stroke (width 0.05) (type solid)) (layer "Edge.Cuts"))
 (gr_line (start 150.5 162) (end 150.5 150.5) (stroke (width 0.05) (type solid)) (layer "Edge.Cuts"))
 (gr_line (start 145 141.1) (end 138.725 141.1) (stroke (width 0.05) (type solid)) (layer "Edge.Cuts"))
 (gr_line (start 138.225 140.6) (end 138.225 140) (stroke (width 0.05) (type solid)) (layer "Edge.Cuts"))
 (gr_line (start 136 162.5) (end 150 162.5) (stroke (width 0.05) (type solid)) (layer "Edge.Cuts"))
 (gr_line (start 150.5 139) (end 150.5 127.5) (stroke (width 0.05) (type solid)) (layer "Edge.Cuts"))
 (gr_line (start 138.375 143.75) (end 145 143.75) (stroke (width 0.05) (type solid)) (layer "Edge.Cuts"))
 (gr_arc (start 135.5 148.62145) (mid 136.341014 146.591014) (end 138.37145 145.75) (stroke (width 0.05) (type solid)) (layer "Edge.Cuts"))
 (gr_arc (start 150.5 116) (mid 150.353553 116.353553) (end 150 116.5) (stroke (width 0.05) (type solid)) (layer "Edge.Cuts"))
 (gr_arc (start 145 118.1) (mid 148.65 121.75) (end 145 125.4) (stroke (width 0.05) (type solid)) (layer "Edge.Cuts"))
 (gr_arc (start 138.725 141.1) (mid 138.371447 140.953553) (end 138.225 140.6) (stroke (width 0.05) (type solid)) (layer "Edge.Cuts"))
 (gr_arc (start 138.225 102.9) (mid 138.371447 102.546447) (end 138.725 102.4) (stroke (width 0.05) (type solid)) (layer "Edge.Cuts"))
 (gr_line (start 145 118.1) (end 138.725 118.1) (stroke (width 0.05) (type solid)) (layer "Edge.Cuts"))
 (gr_arc (start 150 127) (mid 150.353553 127.146447) (end 150.5 127.5) (stroke (width 0.05) (type solid)) (layer "Edge.Cuts"))
 (gr_line (start 138.725 93.5) (end 150 93.5) (stroke (width 0.05) (type solid)) (layer "Edge.Cuts"))
 (gr_line (start 145 145.75) (end 138.37145 145.75) (stroke (width 0.05) (type solid)) (layer "Edge.Cuts"))
 (gr_arc (start 145 143.75) (mid 146 144.75) (end 145 145.75) (stroke (width 0.05) (type solid)) (layer "Edge.Cuts"))
 (gr_arc (start 138.725005 104) (mid 138.371452 103.853553) (end 138.225005 103.5) (stroke (width 0.05) (type solid)) (layer "Edge.Cuts"))
 (gr_line (start 138.225 117.6) (end 138.225 117) (stroke (width 0.05) (type solid)) (layer "Edge.Cuts"))
 (gr_arc (start 145.00001 95.1) (mid 148.65 98.75) (end 145.00001 102.4) (stroke (width 0.05) (type solid)) (layer "Edge.Cuts"))
 (gr_line (start 150 78.5) (end 136 78.5) (stroke (width 0.05) (type solid)) (layer "Edge.Cuts"))
 (gr_line (start 138.22501 103.5) (end 138.225 102.9) (stroke (width 0.05) (type solid)) (layer "Edge.Cuts"))
 (gr_arc (start 150 150) (mid 150.353553 150.146447) (end 150.5 150.5) (stroke (width 0.05) (type solid)) (layer "Edge.Cuts"))
 (gr_arc (start 138.725 118.1) (mid 138.371447 117.953553) (end 138.225 117.6) (stroke (width 0.05) (type solid)) (layer "Edge.Cuts"))
 (gr_line (start 138.37145 97.75) (end 145.00001 97.75) (stroke (width 0.05) (type solid)) (layer "Edge.Cuts"))
 (via (at 138 85.64) (size 1.8) (drill 1.75) (layers "F.Cu" "B.Cu") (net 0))
 (via (at 138 131.64) (size 1.8) (drill 1.75) (layers "F.Cu" "B.Cu") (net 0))
 (via (at 148.16 108.64) (size 1.8) (drill 1.75) (layers "F.Cu" "B.Cu") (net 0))
 (via (at 138 108.64) (size 1.8) (drill 1.75) (layers "F.Cu" "B.Cu") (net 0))
 (via (at 148.16 131.64) (size 1.8) (drill 1.75) (layers "F.Cu" "B.Cu") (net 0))
 (via (at 148.16 154.64) (size 1.8) (drill 1.75) (layers "F.Cu" "B.Cu") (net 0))
 (via (at 138 154.64) (size 1.8) (drill 1.75) (layers "F.Cu" "B.Cu") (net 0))
 (via (at 148.16 85.64) (size 1.8) (drill 1.75) (layers "F.Cu" "B.Cu") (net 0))
 (segment (start 145.708 91.542) (end 144.351 92.899) (width 0.2) (layer "F.Cu") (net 3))
 (segment (start 138.351 92.899) (end 138.25 93) (width 0.2) (layer "F.Cu") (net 3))
 (segment (start 145.708 90.9562) (end 145.708 91.542) (width 0.2) (layer "F.Cu") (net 3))
 (segment (start 144.351 92.899) (end 138.351 92.899) (width 0.2) (layer "F.Cu") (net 3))
 (segment (start 146.5 83.25) (end 146 83.75) (width 0.2) (layer "B.Cu") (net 8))
 (segment (start 146.5 79.925) (end 146.5 83.25) (width 0.2) (layer "B.Cu") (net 8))
 (segment (start 146 83.75) (end 143.75 83.75) (width 0.2) (layer "B.Cu") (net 8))
 (segment (start 143.75 83.75) (end 143.33 84.17) (width 0.2) (layer "B.Cu") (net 8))
 (segment (start 143.33 84.17) (end 143.33 84.94) (width 0.2) (layer "B.Cu") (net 8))
 (segment (start 142.5 84.61) (end 142.5 79.925) (width 0.2) (layer "B.Cu") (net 10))
 (segment (start 142.83 84.94) (end 142.5 84.61) (width 0.2) (layer "B.Cu") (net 10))
 (segment (start 140.2938 89.4562) (end 136.75 93) (width 0.2) (layer "F.Cu") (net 1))
 (segment (start 140.452 89.4562) (end 140.2938 89.4562) (width 0.2) (layer "F.Cu") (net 1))
 (segment (start 136.75 93) (end 136.75 94.25) (width 0.2) (layer "F.Cu") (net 1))
 (segment (start 137.5 93.1257) (end 137.5 93.75) (width 0.2) (layer "F.Cu") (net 2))
 (segment (start 139.6695 90.9562) (end 137.5 93.1257) (width 0.2) (layer "F.Cu") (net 2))
 (segment (start 140.452 90.9562) (end 139.6695 90.9562) (width 0.2) (layer "F.Cu") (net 2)))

